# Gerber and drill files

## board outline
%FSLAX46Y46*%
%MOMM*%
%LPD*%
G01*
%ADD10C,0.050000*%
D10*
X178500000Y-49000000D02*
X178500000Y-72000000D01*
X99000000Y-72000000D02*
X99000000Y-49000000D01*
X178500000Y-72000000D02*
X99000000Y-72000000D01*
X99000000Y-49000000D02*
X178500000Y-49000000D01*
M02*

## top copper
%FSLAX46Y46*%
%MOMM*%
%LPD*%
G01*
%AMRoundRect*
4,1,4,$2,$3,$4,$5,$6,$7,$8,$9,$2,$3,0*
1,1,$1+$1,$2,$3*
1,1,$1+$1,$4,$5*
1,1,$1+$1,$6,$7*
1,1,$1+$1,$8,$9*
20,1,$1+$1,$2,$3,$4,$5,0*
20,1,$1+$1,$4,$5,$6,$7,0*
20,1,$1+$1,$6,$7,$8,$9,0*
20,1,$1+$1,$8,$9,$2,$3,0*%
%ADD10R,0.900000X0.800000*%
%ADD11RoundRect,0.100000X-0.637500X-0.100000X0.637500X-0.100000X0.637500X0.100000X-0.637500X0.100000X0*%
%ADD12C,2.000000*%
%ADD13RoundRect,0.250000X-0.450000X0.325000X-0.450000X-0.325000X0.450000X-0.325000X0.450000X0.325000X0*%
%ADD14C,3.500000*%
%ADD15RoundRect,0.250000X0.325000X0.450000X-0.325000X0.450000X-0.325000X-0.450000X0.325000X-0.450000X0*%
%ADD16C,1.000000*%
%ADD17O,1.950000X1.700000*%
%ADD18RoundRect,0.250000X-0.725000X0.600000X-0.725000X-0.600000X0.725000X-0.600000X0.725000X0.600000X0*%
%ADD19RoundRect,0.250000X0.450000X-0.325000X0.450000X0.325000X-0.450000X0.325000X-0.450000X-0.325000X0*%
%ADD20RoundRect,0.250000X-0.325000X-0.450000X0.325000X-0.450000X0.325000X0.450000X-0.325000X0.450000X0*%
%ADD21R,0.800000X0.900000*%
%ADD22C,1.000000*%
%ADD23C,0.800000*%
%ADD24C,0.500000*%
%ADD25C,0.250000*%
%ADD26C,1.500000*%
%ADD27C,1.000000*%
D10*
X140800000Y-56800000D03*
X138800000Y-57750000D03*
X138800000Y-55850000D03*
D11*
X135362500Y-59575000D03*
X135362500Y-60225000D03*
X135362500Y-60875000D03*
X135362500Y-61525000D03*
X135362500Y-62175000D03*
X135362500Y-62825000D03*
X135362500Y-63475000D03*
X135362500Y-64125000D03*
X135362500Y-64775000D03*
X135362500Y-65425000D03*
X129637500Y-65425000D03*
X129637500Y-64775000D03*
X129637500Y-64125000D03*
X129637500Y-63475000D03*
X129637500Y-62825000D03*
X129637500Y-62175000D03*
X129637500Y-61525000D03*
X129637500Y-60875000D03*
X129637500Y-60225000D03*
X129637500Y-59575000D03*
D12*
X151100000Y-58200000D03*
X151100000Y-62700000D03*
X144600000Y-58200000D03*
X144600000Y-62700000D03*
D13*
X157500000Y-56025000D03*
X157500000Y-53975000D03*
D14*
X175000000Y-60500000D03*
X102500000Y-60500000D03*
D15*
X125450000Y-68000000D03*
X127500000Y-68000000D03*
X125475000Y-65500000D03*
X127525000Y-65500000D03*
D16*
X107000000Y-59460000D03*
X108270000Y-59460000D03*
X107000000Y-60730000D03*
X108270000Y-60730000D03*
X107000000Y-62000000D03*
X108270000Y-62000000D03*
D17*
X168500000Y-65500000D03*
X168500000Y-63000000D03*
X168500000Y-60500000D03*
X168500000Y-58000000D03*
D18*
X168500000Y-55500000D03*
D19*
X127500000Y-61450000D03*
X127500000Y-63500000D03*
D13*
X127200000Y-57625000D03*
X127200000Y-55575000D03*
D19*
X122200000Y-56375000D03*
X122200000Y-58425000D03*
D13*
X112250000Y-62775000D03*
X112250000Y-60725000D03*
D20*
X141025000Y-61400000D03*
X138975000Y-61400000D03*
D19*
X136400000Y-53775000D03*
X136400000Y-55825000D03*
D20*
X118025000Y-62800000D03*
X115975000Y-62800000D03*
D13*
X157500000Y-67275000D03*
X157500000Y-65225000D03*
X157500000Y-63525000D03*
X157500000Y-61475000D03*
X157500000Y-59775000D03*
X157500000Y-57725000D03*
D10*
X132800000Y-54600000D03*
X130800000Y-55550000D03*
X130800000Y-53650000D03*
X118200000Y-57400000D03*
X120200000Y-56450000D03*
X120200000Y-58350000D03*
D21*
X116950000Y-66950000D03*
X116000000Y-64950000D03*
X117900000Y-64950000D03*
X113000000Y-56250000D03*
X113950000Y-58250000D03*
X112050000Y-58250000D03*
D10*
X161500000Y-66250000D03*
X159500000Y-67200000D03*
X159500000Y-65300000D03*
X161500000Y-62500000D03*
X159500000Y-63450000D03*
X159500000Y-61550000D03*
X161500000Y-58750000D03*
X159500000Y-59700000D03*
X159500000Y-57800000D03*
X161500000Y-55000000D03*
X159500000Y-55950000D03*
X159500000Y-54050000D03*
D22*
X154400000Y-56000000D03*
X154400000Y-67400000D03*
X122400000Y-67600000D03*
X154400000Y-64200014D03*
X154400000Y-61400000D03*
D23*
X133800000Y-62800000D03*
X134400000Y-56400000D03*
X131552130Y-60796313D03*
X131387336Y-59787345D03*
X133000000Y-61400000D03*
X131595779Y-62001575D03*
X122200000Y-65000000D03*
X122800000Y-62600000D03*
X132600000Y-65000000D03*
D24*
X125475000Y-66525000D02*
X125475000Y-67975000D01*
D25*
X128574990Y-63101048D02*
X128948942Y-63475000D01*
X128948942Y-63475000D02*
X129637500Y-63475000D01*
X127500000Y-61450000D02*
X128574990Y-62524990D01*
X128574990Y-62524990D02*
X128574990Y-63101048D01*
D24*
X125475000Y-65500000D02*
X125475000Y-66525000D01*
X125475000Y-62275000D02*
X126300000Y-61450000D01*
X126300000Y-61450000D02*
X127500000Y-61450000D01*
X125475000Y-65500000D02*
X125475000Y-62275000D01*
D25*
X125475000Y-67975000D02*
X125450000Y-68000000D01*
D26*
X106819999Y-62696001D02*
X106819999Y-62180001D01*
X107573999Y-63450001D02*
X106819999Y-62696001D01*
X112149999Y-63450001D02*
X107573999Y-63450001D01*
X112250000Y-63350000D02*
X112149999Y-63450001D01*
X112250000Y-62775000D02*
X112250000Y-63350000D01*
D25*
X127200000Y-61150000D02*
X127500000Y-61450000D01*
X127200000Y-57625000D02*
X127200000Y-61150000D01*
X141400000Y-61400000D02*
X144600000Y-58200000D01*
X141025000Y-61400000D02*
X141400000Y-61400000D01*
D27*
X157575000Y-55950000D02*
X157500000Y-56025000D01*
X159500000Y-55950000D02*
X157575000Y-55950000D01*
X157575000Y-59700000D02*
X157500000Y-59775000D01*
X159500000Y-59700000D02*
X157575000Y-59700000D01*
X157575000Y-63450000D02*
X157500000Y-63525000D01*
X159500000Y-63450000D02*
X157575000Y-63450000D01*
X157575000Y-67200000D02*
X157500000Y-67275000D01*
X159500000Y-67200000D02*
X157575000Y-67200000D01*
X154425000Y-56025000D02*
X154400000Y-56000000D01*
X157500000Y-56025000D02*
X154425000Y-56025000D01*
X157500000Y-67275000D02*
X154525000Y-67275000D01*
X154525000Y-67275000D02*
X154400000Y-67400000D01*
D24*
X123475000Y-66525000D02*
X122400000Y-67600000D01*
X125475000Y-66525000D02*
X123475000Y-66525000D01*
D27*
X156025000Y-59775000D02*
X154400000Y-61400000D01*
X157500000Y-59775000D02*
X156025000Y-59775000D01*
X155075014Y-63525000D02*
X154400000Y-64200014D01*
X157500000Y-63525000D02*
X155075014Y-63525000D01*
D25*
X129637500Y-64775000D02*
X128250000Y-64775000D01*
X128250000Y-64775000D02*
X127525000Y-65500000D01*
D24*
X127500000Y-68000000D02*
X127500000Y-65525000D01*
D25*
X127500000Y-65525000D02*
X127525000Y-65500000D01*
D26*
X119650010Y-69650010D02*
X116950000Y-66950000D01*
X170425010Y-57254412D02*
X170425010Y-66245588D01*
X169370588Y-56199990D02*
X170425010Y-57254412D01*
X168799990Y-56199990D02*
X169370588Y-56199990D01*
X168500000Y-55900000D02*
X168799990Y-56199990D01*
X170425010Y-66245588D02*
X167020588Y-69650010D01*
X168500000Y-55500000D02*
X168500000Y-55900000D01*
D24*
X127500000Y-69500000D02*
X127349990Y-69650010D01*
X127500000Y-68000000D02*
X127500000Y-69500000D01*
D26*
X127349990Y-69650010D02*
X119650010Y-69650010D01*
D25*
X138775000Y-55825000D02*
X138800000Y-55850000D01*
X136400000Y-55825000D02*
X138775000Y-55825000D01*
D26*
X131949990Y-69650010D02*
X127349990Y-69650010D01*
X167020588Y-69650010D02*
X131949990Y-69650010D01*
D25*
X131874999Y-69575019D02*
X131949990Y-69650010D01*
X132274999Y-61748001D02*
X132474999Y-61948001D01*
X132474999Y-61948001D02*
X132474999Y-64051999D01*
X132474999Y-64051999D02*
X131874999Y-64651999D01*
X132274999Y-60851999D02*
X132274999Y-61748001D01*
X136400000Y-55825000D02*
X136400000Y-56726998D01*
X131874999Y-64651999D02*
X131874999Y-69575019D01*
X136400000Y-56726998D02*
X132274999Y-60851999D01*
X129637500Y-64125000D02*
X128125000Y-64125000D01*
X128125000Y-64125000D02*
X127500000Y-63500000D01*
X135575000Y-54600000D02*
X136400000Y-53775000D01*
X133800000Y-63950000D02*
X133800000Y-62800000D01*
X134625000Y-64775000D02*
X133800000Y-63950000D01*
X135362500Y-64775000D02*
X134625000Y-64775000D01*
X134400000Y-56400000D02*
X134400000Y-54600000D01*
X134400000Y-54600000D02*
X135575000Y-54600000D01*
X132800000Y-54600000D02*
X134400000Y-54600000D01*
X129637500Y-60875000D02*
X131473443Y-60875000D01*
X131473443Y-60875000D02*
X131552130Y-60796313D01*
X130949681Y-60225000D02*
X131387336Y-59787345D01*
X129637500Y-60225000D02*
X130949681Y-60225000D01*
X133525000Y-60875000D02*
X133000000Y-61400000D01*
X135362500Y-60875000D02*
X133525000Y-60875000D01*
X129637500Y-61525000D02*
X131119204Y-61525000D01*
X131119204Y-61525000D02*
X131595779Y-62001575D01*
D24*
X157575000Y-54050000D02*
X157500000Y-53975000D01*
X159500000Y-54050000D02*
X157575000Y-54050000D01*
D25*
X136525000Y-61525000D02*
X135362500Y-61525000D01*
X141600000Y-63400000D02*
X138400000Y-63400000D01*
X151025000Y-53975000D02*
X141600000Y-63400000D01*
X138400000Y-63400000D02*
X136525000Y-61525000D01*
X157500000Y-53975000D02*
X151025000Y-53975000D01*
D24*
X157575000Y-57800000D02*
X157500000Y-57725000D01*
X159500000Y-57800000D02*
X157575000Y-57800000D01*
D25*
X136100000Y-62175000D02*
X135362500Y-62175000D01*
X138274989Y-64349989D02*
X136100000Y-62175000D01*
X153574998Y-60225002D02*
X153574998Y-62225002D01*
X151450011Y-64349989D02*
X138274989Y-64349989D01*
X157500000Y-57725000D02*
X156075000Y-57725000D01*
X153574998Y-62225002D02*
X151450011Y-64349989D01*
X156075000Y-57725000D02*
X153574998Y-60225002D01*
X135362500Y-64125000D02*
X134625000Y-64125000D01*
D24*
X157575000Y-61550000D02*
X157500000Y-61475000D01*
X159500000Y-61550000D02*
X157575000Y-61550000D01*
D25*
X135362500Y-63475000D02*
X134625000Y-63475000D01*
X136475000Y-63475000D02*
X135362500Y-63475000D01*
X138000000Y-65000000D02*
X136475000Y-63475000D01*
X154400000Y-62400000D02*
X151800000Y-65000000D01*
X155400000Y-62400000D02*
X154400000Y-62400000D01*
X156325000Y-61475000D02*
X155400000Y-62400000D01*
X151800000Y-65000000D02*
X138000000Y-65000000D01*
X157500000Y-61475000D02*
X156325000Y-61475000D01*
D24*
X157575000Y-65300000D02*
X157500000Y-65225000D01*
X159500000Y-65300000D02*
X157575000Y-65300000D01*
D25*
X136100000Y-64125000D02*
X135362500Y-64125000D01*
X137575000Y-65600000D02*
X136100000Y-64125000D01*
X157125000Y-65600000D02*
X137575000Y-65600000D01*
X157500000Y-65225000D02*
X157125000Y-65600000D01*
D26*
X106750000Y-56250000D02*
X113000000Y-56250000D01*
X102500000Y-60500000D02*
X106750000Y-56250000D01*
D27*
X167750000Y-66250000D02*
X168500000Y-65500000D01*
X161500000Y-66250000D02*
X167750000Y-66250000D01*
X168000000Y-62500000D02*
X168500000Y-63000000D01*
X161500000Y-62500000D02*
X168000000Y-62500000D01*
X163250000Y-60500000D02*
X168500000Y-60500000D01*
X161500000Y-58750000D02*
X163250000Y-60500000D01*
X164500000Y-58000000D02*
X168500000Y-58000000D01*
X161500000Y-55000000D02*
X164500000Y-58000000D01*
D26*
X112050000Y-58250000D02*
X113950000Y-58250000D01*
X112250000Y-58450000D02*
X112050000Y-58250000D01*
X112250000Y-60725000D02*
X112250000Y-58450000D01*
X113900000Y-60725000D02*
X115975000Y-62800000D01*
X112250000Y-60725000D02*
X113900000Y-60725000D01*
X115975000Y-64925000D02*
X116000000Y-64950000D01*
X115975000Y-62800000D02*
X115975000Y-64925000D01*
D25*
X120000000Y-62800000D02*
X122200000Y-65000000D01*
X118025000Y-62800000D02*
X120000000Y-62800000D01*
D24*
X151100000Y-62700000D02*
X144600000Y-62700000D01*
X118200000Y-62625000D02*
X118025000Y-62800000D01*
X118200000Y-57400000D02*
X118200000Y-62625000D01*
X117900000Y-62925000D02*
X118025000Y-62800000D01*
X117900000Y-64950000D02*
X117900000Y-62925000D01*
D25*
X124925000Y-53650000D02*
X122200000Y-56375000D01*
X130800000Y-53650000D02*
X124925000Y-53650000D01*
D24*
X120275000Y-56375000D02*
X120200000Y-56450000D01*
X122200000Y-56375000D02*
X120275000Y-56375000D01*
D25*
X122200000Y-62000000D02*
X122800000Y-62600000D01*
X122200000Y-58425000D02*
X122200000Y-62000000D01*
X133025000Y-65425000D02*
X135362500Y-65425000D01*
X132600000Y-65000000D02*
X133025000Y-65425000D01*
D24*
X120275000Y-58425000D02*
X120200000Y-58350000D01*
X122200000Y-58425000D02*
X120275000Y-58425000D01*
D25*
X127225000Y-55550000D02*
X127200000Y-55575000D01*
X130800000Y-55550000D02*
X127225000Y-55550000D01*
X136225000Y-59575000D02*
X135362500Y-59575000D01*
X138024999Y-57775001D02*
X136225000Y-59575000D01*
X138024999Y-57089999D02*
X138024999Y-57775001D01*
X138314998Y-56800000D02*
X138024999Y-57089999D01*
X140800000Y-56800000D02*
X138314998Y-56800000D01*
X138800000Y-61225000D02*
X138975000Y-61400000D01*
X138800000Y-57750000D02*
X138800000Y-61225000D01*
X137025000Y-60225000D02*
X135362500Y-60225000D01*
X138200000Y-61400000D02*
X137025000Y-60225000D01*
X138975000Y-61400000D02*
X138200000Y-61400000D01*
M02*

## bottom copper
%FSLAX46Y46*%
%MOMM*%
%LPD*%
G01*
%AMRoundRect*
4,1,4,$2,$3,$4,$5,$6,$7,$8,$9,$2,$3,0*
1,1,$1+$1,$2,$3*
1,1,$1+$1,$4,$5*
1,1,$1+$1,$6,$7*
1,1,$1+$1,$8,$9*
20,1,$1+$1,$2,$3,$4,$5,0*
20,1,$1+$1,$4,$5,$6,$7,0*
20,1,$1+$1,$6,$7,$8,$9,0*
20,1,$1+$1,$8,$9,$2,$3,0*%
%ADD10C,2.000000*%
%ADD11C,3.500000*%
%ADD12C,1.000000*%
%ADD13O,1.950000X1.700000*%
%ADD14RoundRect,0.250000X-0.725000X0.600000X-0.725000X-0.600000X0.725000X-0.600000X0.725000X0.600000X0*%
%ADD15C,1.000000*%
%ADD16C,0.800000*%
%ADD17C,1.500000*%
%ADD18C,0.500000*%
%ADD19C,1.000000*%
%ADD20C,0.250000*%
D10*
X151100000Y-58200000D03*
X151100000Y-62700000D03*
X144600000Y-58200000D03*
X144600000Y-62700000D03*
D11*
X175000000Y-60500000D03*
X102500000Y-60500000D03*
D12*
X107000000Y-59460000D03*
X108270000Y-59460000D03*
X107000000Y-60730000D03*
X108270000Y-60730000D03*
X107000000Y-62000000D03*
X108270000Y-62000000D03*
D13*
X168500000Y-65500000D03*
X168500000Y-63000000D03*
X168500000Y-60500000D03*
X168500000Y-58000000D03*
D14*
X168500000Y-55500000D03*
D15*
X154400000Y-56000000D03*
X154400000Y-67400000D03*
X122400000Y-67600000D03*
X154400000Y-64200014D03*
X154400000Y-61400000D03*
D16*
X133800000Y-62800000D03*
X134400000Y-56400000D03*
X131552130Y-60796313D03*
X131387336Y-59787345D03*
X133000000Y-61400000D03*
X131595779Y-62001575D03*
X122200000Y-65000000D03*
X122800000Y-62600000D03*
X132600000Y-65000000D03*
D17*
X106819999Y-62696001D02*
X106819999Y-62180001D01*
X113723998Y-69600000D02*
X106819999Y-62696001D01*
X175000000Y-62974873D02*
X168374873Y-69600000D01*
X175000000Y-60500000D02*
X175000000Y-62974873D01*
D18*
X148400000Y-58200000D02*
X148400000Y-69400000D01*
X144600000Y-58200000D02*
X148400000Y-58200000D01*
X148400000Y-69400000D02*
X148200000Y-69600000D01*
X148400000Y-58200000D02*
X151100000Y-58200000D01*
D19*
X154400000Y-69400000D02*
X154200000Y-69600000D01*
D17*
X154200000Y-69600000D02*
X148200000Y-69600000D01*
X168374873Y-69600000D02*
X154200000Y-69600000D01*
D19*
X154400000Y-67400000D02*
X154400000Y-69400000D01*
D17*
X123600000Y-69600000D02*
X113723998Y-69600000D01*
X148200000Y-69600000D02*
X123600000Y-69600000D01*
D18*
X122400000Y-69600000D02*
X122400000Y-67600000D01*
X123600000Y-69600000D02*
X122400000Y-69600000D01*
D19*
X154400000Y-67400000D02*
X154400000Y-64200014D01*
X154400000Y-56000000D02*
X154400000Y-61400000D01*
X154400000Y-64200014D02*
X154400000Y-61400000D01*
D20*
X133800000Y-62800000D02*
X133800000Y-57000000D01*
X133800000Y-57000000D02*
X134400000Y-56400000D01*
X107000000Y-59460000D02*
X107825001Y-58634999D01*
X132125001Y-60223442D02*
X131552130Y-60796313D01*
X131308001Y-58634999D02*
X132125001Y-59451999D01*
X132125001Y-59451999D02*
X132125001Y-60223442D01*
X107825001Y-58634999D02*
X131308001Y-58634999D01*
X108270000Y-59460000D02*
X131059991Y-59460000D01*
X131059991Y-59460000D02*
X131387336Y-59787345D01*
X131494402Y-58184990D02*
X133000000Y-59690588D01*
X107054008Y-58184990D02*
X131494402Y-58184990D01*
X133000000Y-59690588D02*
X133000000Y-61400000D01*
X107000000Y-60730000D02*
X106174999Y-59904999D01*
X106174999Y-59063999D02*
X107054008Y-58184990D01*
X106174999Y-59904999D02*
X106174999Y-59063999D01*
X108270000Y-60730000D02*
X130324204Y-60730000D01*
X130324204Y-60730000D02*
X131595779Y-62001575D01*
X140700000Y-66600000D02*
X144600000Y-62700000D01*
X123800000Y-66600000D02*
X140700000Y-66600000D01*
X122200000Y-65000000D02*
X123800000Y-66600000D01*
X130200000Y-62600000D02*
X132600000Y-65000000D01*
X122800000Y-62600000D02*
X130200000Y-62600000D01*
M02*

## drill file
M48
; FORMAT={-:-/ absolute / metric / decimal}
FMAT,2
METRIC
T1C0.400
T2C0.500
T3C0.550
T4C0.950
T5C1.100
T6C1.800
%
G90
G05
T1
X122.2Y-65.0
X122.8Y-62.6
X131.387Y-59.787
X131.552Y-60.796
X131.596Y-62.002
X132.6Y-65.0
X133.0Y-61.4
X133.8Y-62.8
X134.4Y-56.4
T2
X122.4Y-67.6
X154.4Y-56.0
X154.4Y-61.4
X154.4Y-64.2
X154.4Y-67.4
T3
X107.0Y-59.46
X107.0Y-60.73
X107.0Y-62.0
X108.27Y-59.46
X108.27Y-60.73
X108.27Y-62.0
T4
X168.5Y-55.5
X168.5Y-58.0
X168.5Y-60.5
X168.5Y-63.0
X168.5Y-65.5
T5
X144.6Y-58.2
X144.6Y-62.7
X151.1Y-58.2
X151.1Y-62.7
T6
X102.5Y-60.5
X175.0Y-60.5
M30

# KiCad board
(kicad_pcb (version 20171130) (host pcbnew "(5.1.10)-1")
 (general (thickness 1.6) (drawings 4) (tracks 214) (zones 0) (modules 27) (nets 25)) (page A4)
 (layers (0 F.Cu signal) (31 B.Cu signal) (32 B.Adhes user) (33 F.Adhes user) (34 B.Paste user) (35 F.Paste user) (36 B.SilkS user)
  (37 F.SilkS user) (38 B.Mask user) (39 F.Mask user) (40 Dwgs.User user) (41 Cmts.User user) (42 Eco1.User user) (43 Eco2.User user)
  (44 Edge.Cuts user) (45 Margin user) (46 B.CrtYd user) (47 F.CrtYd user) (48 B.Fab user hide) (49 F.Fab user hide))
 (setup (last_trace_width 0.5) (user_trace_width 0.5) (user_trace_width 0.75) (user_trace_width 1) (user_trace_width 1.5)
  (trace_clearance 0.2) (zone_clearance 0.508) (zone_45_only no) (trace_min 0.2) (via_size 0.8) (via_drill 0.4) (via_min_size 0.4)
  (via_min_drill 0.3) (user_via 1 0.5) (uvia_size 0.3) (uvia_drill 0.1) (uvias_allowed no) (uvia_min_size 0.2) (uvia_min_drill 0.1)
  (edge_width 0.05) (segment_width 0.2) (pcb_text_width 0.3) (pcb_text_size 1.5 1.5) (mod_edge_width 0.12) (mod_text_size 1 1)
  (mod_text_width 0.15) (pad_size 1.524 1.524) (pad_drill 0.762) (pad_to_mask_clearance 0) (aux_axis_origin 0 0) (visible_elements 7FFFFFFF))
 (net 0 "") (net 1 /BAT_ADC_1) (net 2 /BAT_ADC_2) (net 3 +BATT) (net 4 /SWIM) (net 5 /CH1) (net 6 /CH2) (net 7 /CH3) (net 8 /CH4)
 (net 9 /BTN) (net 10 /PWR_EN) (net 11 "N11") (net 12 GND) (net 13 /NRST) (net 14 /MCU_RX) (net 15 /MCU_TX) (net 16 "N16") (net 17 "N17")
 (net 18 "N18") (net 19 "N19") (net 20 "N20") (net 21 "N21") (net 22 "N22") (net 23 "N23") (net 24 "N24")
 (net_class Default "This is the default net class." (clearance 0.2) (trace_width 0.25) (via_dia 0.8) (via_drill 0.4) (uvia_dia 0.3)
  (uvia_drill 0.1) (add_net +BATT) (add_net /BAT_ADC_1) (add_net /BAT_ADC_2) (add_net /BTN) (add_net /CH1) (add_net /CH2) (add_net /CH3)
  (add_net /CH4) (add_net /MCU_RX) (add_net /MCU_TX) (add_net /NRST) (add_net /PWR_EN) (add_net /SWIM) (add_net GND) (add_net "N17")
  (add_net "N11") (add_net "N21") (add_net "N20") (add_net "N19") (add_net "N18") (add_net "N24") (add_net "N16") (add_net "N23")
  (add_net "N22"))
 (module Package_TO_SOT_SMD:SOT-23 (layer F.Cu) (at 139.8 56.8)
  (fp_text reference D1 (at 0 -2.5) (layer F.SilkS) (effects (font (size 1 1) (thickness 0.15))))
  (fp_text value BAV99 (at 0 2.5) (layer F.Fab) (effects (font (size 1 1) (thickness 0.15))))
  (pad 3 smd rect (at 1 0) (size 0.9 0.8) (layers F.Cu F.Paste F.Mask) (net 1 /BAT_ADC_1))
  (pad 2 smd rect (at -1 0.95) (size 0.9 0.8) (layers F.Cu F.Paste F.Mask) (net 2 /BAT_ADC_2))
  (pad 1 smd rect (at -1 -0.95) (size 0.9 0.8) (layers F.Cu F.Paste F.Mask) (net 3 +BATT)))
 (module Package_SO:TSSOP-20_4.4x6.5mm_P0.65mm (layer F.Cu) (at 132.5 62.5)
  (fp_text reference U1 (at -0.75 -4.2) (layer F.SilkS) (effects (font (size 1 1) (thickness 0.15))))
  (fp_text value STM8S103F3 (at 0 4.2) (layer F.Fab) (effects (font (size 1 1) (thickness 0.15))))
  (pad 20 smd roundrect (at 2.8625 -2.925) (size 1.475 0.4) (layers F.Cu F.Paste F.Mask) (roundrect_rratio 0.25) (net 1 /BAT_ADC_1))
  (pad 19 smd roundrect (at 2.8625 -2.275) (size 1.475 0.4) (layers F.Cu F.Paste F.Mask) (roundrect_rratio 0.25) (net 2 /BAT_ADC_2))
  (pad 18 smd roundrect (at 2.8625 -1.625) (size 1.475 0.4) (layers F.Cu F.Paste F.Mask) (roundrect_rratio 0.25) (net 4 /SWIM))
  (pad 17 smd roundrect (at 2.8625 -0.975) (size 1.475 0.4) (layers F.Cu F.Paste F.Mask) (roundrect_rratio 0.25) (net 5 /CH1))
  (pad 16 smd roundrect (at 2.8625 -0.325) (size 1.475 0.4) (layers F.Cu F.Paste F.Mask) (roundrect_rratio 0.25) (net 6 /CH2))
  (pad 15 smd roundrect (at 2.8625 0.325) (size 1.475 0.4) (layers F.Cu F.Paste F.Mask) (roundrect_rratio 0.25))
  (pad 14 smd roundrect (at 2.8625 0.975) (size 1.475 0.4) (layers F.Cu F.Paste F.Mask) (roundrect_rratio 0.25) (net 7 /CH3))
  (pad 13 smd roundrect (at 2.8625 1.625) (size 1.475 0.4) (layers F.Cu F.Paste F.Mask) (roundrect_rratio 0.25) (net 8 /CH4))
  (pad 12 smd roundrect (at 2.8625 2.275) (size 1.475 0.4) (layers F.Cu F.Paste F.Mask) (roundrect_rratio 0.25) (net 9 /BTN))
  (pad 11 smd roundrect (at 2.8625 2.925) (size 1.475 0.4) (layers F.Cu F.Paste F.Mask) (roundrect_rratio 0.25) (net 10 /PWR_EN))
  (pad 10 smd roundrect (at -2.8625 2.925) (size 1.475 0.4) (layers F.Cu F.Paste F.Mask) (roundrect_rratio 0.25))
  (pad 9 smd roundrect (at -2.8625 2.275) (size 1.475 0.4) (layers F.Cu F.Paste F.Mask) (roundrect_rratio 0.25) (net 3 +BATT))
  (pad 8 smd roundrect (at -2.8625 1.625) (size 1.475 0.4) (layers F.Cu F.Paste F.Mask) (roundrect_rratio 0.25) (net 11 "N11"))
  (pad 7 smd roundrect (at -2.8625 0.975) (size 1.475 0.4) (layers F.Cu F.Paste F.Mask) (roundrect_rratio 0.25) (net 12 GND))
  (pad 6 smd roundrect (at -2.8625 0.325) (size 1.475 0.4) (layers F.Cu F.Paste F.Mask) (roundrect_rratio 0.25))
  (pad 5 smd roundrect (at -2.8625 -0.325) (size 1.475 0.4) (layers F.Cu F.Paste F.Mask) (roundrect_rratio 0.25))
  (pad 4 smd roundrect (at -2.8625 -0.975) (size 1.475 0.4) (layers F.Cu F.Paste F.Mask) (roundrect_rratio 0.25) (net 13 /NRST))
  (pad 3 smd roundrect (at -2.8625 -1.625) (size 1.475 0.4) (layers F.Cu F.Paste F.Mask) (roundrect_rratio 0.25) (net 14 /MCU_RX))
  (pad 2 smd roundrect (at -2.8625 -2.275) (size 1.475 0.4) (layers F.Cu F.Paste F.Mask) (roundrect_rratio 0.25) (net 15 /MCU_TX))
  (pad 1 smd roundrect (at -2.8625 -2.925) (size 1.475 0.4) (layers F.Cu F.Paste F.Mask) (roundrect_rratio 0.25)))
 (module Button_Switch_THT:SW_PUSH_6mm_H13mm (layer F.Cu) (at 144.6 58.2)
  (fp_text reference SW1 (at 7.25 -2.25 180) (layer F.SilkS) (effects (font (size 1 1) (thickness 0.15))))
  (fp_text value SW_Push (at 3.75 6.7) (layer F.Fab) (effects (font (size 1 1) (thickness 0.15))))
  (pad 1 thru_hole circle (at 6.5 0 90) (size 2 2) (drill 1.1) (layers *.Cu *.Mask) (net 12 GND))
  (pad 2 thru_hole circle (at 6.5 4.5 90) (size 2 2) (drill 1.1) (layers *.Cu *.Mask) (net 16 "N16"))
  (pad 1 thru_hole circle (at 0 0 90) (size 2 2) (drill 1.1) (layers *.Cu *.Mask) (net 12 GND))
  (pad 2 thru_hole circle (at 0 4.5 90) (size 2 2) (drill 1.1) (layers *.Cu *.Mask) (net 16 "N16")))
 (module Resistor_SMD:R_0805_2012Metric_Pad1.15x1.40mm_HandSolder (layer F.Cu) (at 157.5 55 270)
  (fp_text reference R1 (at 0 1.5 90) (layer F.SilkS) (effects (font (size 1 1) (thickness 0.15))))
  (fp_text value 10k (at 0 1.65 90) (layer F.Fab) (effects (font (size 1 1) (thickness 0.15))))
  (pad 2 smd roundrect (at 1.025 0 270) (size 1.15 1.4) (layers F.Cu F.Paste F.Mask) (roundrect_rratio 0.217391) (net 12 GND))
  (pad 1 smd roundrect (at -1.025 0 270) (size 1.15 1.4) (layers F.Cu F.Paste F.Mask) (roundrect_rratio 0.217391) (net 5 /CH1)))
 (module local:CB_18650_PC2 (layer B.Cu) (at 100 71)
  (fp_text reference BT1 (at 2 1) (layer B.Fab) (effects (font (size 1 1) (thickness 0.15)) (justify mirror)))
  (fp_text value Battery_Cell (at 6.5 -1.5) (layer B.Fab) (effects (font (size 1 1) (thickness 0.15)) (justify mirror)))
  (pad 2 thru_hole circle (at 75 -10.5) (size 3.5 3.5) (drill 1.8) (layers *.Cu *.Mask) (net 12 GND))
  (pad 1 thru_hole circle (at 2.5 -10.5) (size 3.5 3.5) (drill 1.8) (layers *.Cu *.Mask) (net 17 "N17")))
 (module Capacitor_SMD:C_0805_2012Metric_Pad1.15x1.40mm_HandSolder (layer F.Cu) (at 126.475 68 180)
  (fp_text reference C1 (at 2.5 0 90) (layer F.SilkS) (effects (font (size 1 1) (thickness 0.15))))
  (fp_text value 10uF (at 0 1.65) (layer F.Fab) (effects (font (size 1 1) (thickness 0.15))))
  (pad 2 smd roundrect (at 1.025 0 180) (size 1.15 1.4) (layers F.Cu F.Paste F.Mask) (roundrect_rratio 0.217391) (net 12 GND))
  (pad 1 smd roundrect (at -1.025 0 180) (size 1.15 1.4) (layers F.Cu F.Paste F.Mask) (roundrect_rratio 0.217391) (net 3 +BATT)))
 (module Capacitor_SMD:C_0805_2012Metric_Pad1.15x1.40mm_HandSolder (layer F.Cu) (at 126.5 65.5 180)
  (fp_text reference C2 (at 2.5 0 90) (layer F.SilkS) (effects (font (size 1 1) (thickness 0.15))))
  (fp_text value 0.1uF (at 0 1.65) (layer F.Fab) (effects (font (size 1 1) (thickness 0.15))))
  (pad 2 smd roundrect (at 1.025 0 180) (size 1.15 1.4) (layers F.Cu F.Paste F.Mask) (roundrect_rratio 0.217391) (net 12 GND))
  (pad 1 smd roundrect (at -1.025 0 180) (size 1.15 1.4) (layers F.Cu F.Paste F.Mask) (roundrect_rratio 0.217391) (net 3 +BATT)))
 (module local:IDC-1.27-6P (layer F.Cu) (at 107 62 90)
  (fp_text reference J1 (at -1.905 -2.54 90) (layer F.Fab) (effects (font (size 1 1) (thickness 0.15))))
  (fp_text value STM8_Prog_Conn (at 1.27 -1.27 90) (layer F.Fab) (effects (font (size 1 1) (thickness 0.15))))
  (pad 6 thru_hole circle (at 2.54 0 90) (size 1 1) (drill 0.55) (layers *.Cu *.Mask) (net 14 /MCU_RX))
  (pad 5 thru_hole circle (at 2.54 1.27 90) (size 1 1) (drill 0.55) (layers *.Cu *.Mask) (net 15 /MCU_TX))
  (pad 4 thru_hole circle (at 1.27 0 90) (size 1 1) (drill 0.55) (layers *.Cu *.Mask) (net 4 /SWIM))
  (pad 3 thru_hole circle (at 1.27 1.27 90) (size 1 1) (drill 0.55) (layers *.Cu *.Mask) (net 13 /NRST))
  (pad 2 thru_hole circle (at 0 0 90) (size 1 1) (drill 0.55) (layers *.Cu *.Mask) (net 12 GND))
  (pad 1 thru_hole circle (at 0 1.27 90) (size 1 1) (drill 0.55) (layers *.Cu *.Mask)))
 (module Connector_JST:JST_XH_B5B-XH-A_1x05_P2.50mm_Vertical (layer F.Cu) (at 168.5 55.5 270)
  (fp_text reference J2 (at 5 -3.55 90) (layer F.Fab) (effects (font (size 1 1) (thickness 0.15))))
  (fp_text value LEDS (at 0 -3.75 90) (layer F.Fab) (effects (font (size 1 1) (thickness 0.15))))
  (pad 5 thru_hole oval (at 10 0 270) (size 1.7 1.95) (drill 0.95) (layers *.Cu *.Mask) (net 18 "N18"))
  (pad 4 thru_hole oval (at 7.5 0 270) (size 1.7 1.95) (drill 0.95) (layers *.Cu *.Mask) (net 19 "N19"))
  (pad 3 thru_hole oval (at 5 0 270) (size 1.7 1.95) (drill 0.95) (layers *.Cu *.Mask) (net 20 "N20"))
  (pad 2 thru_hole oval (at 2.5 0 270) (size 1.7 1.95) (drill 0.95) (layers *.Cu *.Mask) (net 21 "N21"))
  (pad 1 thru_hole roundrect (at 0 0 270) (size 1.7 1.95) (drill 0.95) (layers *.Cu *.Mask) (roundrect_rratio 0.147059) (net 3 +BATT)))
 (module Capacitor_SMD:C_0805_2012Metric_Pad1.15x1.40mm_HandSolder (layer F.Cu) (at 127.5 62.475 90)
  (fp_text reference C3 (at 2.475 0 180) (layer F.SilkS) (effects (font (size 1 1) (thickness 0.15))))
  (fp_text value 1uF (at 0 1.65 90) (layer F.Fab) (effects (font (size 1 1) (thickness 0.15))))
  (pad 2 smd roundrect (at 1.025 0 90) (size 1.15 1.4) (layers F.Cu F.Paste F.Mask) (roundrect_rratio 0.217391) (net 12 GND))
  (pad 1 smd roundrect (at -1.025 0 90) (size 1.15 1.4) (layers F.Cu F.Paste F.Mask) (roundrect_rratio 0.217391) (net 11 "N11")))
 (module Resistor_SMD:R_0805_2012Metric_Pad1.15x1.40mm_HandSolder (layer F.Cu) (at 127.2 56.6 270)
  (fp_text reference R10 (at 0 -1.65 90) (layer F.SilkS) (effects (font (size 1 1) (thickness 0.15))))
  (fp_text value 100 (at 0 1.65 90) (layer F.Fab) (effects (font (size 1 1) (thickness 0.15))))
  (pad 2 smd roundrect (at 1.025 0 270) (size 1.15 1.4) (layers F.Cu F.Paste F.Mask) (roundrect_rratio 0.217391) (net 12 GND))
  (pad 1 smd roundrect (at -1.025 0 270) (size 1.15 1.4) (layers F.Cu F.Paste F.Mask) (roundrect_rratio 0.217391) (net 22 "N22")))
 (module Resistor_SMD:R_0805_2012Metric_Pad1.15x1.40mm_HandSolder (layer F.Cu) (at 122.2 57.4 90)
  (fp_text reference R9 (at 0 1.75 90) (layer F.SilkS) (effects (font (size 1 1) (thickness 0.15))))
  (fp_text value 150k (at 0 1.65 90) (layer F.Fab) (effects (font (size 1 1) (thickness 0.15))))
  (pad 2 smd roundrect (at 1.025 0 90) (size 1.15 1.4) (layers F.Cu F.Paste F.Mask) (roundrect_rratio 0.217391) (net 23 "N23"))
  (pad 1 smd roundrect (at -1.025 0 90) (size 1.15 1.4) (layers F.Cu F.Paste F.Mask) (roundrect_rratio 0.217391) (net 10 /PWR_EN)))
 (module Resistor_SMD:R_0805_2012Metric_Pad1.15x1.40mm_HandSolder (layer F.Cu) (at 112.25 61.75 270)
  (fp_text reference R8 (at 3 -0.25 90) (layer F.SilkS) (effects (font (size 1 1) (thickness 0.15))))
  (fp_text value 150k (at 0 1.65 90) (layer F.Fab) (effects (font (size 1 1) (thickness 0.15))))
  (pad 2 smd roundrect (at 1.025 0 270) (size 1.15 1.4) (layers F.Cu F.Paste F.Mask) (roundrect_rratio 0.217391) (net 12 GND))
  (pad 1 smd roundrect (at -1.025 0 270) (size 1.15 1.4) (layers F.Cu F.Paste F.Mask) (roundrect_rratio 0.217391) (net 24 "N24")))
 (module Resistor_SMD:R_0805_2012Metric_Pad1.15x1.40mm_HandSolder (layer F.Cu) (at 140 61.4)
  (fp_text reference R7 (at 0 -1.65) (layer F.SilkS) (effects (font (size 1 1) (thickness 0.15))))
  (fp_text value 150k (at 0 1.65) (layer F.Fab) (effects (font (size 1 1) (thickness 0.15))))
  (pad 2 smd roundrect (at 1.025 0) (size 1.15 1.4) (layers F.Cu F.Paste F.Mask) (roundrect_rratio 0.217391) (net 12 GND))
  (pad 1 smd roundrect (at -1.025 0) (size 1.15 1.4) (layers F.Cu F.Paste F.Mask) (roundrect_rratio 0.217391) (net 2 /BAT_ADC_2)))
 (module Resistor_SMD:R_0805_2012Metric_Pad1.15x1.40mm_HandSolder (layer F.Cu) (at 136.4 54.8 90)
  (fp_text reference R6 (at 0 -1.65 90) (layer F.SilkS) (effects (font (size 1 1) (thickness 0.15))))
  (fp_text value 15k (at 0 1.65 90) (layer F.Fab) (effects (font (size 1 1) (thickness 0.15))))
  (pad 2 smd roundrect (at 1.025 0 90) (size 1.15 1.4) (layers F.Cu F.Paste F.Mask) (roundrect_rratio 0.217391) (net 9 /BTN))
  (pad 1 smd roundrect (at -1.025 0 90) (size 1.15 1.4) (layers F.Cu F.Paste F.Mask) (roundrect_rratio 0.217391) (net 3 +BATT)))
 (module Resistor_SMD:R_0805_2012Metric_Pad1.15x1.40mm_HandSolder (layer F.Cu) (at 117 62.8)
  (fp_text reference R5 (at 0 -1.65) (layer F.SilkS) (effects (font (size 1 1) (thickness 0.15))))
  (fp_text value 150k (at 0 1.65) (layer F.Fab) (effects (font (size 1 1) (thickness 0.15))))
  (pad 2 smd roundrect (at 1.025 0) (size 1.15 1.4) (layers F.Cu F.Paste F.Mask) (roundrect_rratio 0.217391) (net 16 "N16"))
  (pad 1 smd roundrect (at -1.025 0) (size 1.15 1.4) (layers F.Cu F.Paste F.Mask) (roundrect_rratio 0.217391) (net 24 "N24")))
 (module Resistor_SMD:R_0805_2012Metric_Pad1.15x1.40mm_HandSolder (layer F.Cu) (at 157.5 66.25 270)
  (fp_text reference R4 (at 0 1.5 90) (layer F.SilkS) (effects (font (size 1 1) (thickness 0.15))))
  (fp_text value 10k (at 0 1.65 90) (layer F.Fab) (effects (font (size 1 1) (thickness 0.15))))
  (pad 2 smd roundrect (at 1.025 0 270) (size 1.15 1.4) (layers F.Cu F.Paste F.Mask) (roundrect_rratio 0.217391) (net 12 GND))
  (pad 1 smd roundrect (at -1.025 0 270) (size 1.15 1.4) (layers F.Cu F.Paste F.Mask) (roundrect_rratio 0.217391) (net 8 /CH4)))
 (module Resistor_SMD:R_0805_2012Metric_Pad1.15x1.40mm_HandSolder (layer F.Cu) (at 157.5 62.5 270)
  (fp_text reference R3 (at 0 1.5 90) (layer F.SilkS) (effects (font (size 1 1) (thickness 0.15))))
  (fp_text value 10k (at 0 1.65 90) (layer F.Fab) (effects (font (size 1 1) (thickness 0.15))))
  (pad 2 smd roundrect (at 1.025 0 270) (size 1.15 1.4) (layers F.Cu F.Paste F.Mask) (roundrect_rratio 0.217391) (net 12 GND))
  (pad 1 smd roundrect (at -1.025 0 270) (size 1.15 1.4) (layers F.Cu F.Paste F.Mask) (roundrect_rratio 0.217391) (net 7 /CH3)))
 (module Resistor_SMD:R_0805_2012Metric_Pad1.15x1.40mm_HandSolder (layer F.Cu) (at 157.5 58.75 270)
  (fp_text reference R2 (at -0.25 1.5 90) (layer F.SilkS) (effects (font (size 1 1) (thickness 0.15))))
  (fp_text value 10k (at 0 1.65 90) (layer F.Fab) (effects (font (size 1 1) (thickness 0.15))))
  (pad 2 smd roundrect (at 1.025 0 270) (size 1.15 1.4) (layers F.Cu F.Paste F.Mask) (roundrect_rratio 0.217391) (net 12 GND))
  (pad 1 smd roundrect (at -1.025 0 270) (size 1.15 1.4) (layers F.Cu F.Paste F.Mask) (roundrect_rratio 0.217391) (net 6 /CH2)))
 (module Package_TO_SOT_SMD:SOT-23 (layer F.Cu) (at 131.8 54.6)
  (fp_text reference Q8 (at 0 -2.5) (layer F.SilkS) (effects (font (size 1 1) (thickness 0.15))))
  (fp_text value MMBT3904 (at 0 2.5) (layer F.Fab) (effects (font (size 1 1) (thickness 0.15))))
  (pad 3 smd rect (at 1 0) (size 0.9 0.8) (layers F.Cu F.Paste F.Mask) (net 9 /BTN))
  (pad 2 smd rect (at -1 0.95) (size 0.9 0.8) (layers F.Cu F.Paste F.Mask) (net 22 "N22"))
  (pad 1 smd rect (at -1 -0.95) (size 0.9 0.8) (layers F.Cu F.Paste F.Mask) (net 23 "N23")))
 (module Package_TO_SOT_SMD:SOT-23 (layer F.Cu) (at 119.2 57.4 180)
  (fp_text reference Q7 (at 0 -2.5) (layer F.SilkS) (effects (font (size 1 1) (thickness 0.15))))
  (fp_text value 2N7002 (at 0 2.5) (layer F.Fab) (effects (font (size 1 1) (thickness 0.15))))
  (pad 3 smd rect (at 1 0 180) (size 0.9 0.8) (layers F.Cu F.Paste F.Mask) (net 16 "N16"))
  (pad 2 smd rect (at -1 0.95 180) (size 0.9 0.8) (layers F.Cu F.Paste F.Mask) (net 23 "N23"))
  (pad 1 smd rect (at -1 -0.95 180) (size 0.9 0.8) (layers F.Cu F.Paste F.Mask) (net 10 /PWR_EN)))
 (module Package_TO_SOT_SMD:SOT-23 (layer F.Cu) (at 116.95 65.95 270)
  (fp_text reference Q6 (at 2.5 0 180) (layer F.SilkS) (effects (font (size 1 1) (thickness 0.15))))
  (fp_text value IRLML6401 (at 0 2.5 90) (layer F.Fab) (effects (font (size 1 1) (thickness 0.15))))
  (pad 3 smd rect (at 1 0 270) (size 0.9 0.8) (layers F.Cu F.Paste F.Mask) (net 3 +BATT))
  (pad 2 smd rect (at -1 0.95 270) (size 0.9 0.8) (layers F.Cu F.Paste F.Mask) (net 24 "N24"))
  (pad 1 smd rect (at -1 -0.95 270) (size 0.9 0.8) (layers F.Cu F.Paste F.Mask) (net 16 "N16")))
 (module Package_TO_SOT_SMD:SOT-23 (layer F.Cu) (at 113 57.25 90)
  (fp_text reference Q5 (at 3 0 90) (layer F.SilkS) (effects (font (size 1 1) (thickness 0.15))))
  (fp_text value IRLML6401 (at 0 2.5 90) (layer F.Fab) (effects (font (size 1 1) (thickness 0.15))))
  (pad 3 smd rect (at 1 0 90) (size 0.9 0.8) (layers F.Cu F.Paste F.Mask) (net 17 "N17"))
  (pad 2 smd rect (at -1 0.95 90) (size 0.9 0.8) (layers F.Cu F.Paste F.Mask) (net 24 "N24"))
  (pad 1 smd rect (at -1 -0.95 90) (size 0.9 0.8) (layers F.Cu F.Paste F.Mask) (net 24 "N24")))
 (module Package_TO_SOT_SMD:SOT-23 (layer F.Cu) (at 160.5 66.25)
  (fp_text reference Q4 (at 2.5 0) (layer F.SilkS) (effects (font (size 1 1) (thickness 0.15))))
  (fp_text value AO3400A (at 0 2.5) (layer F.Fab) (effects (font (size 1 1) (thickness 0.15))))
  (pad 3 smd rect (at 1 0) (size 0.9 0.8) (layers F.Cu F.Paste F.Mask) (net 18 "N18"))
  (pad 2 smd rect (at -1 0.95) (size 0.9 0.8) (layers F.Cu F.Paste F.Mask) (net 12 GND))
  (pad 1 smd rect (at -1 -0.95) (size 0.9 0.8) (layers F.Cu F.Paste F.Mask) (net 8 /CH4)))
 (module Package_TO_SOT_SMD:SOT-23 (layer F.Cu) (at 160.5 62.5)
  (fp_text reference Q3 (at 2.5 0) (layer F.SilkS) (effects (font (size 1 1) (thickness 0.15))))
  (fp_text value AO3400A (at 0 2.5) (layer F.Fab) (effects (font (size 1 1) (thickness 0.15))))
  (pad 3 smd rect (at 1 0) (size 0.9 0.8) (layers F.Cu F.Paste F.Mask) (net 19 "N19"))
  (pad 2 smd rect (at -1 0.95) (size 0.9 0.8) (layers F.Cu F.Paste F.Mask) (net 12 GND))
  (pad 1 smd rect (at -1 -0.95) (size 0.9 0.8) (layers F.Cu F.Paste F.Mask) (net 7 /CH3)))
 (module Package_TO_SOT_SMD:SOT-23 (layer F.Cu) (at 160.5 58.75)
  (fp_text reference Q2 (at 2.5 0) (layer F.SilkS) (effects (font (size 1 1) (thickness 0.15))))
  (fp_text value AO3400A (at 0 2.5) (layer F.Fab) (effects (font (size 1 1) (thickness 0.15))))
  (pad 3 smd rect (at 1 0) (size 0.9 0.8) (layers F.Cu F.Paste F.Mask) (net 20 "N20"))
  (pad 2 smd rect (at -1 0.95) (size 0.9 0.8) (layers F.Cu F.Paste F.Mask) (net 12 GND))
  (pad 1 smd rect (at -1 -0.95) (size 0.9 0.8) (layers F.Cu F.Paste F.Mask) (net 6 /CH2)))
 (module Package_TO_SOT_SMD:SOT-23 (layer F.Cu) (at 160.5 55)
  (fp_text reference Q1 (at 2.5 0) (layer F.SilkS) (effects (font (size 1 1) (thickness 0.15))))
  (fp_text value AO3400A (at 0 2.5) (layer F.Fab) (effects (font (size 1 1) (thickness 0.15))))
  (pad 3 smd rect (at 1 0) (size 0.9 0.8) (layers F.Cu F.Paste F.Mask) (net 21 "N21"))
  (pad 2 smd rect (at -1 0.95) (size 0.9 0.8) (layers F.Cu F.Paste F.Mask) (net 12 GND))
  (pad 1 smd rect (at -1 -0.95) (size 0.9 0.8) (layers F.Cu F.Paste F.Mask) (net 5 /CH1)))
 (gr_line (start 178.5 49) (end 178.5 72) (layer Edge.Cuts) (width 0.05))
 (gr_line (start 99 72) (end 99 49) (layer Edge.Cuts) (width 0.05))
 (gr_line (start 178.5 72) (end 99 72) (layer Edge.Cuts) (width 0.05))
 (gr_line (start 99 49) (end 178.5 49) (layer Edge.Cuts) (width 0.05))
 (segment (start 125.475 66.525) (end 125.475 67.975) (width 0.5) (layer F.Cu) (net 12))
 (segment (start 128.57499 63.101048) (end 128.948942 63.475) (width 0.25) (layer F.Cu) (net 12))
 (segment (start 128.948942 63.475) (end 129.6375 63.475) (width 0.25) (layer F.Cu) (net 12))
 (segment (start 127.5 61.45) (end 128.57499 62.52499) (width 0.25) (layer F.Cu) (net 12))
 (segment (start 128.57499 62.52499) (end 128.57499 63.101048) (width 0.25) (layer F.Cu) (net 12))
 (segment (start 125.475 65.5) (end 125.475 66.525) (width 0.5) (layer F.Cu) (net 12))
 (segment (start 125.475 62.275) (end 126.3 61.45) (width 0.5) (layer F.Cu) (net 12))
 (segment (start 126.3 61.45) (end 127.5 61.45) (width 0.5) (layer F.Cu) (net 12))
 (segment (start 125.475 65.5) (end 125.475 62.275) (width 0.5) (layer F.Cu) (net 12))
 (segment (start 125.475 67.975) (end 125.45 68) (width 0.25) (layer F.Cu) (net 12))
 (segment (start 106.819999 62.696001) (end 106.819999 62.180001) (width 1.5) (layer F.Cu) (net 12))
 (segment (start 107.573999 63.450001) (end 106.819999 62.696001) (width 1.5) (layer F.Cu) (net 12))
 (segment (start 112.149999 63.450001) (end 107.573999 63.450001) (width 1.5) (layer F.Cu) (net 12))
 (segment (start 112.25 63.35) (end 112.149999 63.450001) (width 1.5) (layer F.Cu) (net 12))
 (segment (start 112.25 62.775) (end 112.25 63.35) (width 1.5) (layer F.Cu) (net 12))
 (segment (start 106.819999 62.696001) (end 106.819999 62.180001) (width 1.5) (layer B.Cu) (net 12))
 (segment (start 113.723998 69.6) (end 106.819999 62.696001) (width 1.5) (layer B.Cu) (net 12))
 (segment (start 175 62.974873) (end 168.374873 69.6) (width 1.5) (layer B.Cu) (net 12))
 (segment (start 175 60.5) (end 175 62.974873) (width 1.5) (layer B.Cu) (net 12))
 (segment (start 127.2 61.15) (end 127.5 61.45) (width 0.25) (layer F.Cu) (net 12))
 (segment (start 127.2 57.625) (end 127.2 61.15) (width 0.25) (layer F.Cu) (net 12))
 (segment (start 148.4 58.2) (end 148.4 69.4) (width 0.5) (layer B.Cu) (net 12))
 (segment (start 144.6 58.2) (end 148.4 58.2) (width 0.5) (layer B.Cu) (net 12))
 (segment (start 148.4 69.4) (end 148.2 69.6) (width 0.5) (layer B.Cu) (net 12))
 (segment (start 148.4 58.2) (end 151.1 58.2) (width 0.5) (layer B.Cu) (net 12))
 (segment (start 141.4 61.4) (end 144.6 58.2) (width 0.25) (layer F.Cu) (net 12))
 (segment (start 141.025 61.4) (end 141.4 61.4) (width 0.25) (layer F.Cu) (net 12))
 (segment (start 157.575 55.95) (end 157.5 56.025) (width 1) (layer F.Cu) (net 12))
 (segment (start 159.5 55.95) (end 157.575 55.95) (width 1) (layer F.Cu) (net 12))
 (segment (start 157.575 59.7) (end 157.5 59.775) (width 1) (layer F.Cu) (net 12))
 (segment (start 159.5 59.7) (end 157.575 59.7) (width 1) (layer F.Cu) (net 12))
 (segment (start 157.575 63.45) (end 157.5 63.525) (width 1) (layer F.Cu) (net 12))
 (segment (start 159.5 63.45) (end 157.575 63.45) (width 1) (layer F.Cu) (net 12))
 (segment (start 157.575 67.2) (end 157.5 67.275) (width 1) (layer F.Cu) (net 12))
 (segment (start 159.5 67.2) (end 157.575 67.2) (width 1) (layer F.Cu) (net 12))
 (via (at 154.4 56) (size 1) (drill 0.5) (layers F.Cu B.Cu) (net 12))
 (segment (start 154.425 56.025) (end 154.4 56) (width 1) (layer F.Cu) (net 12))
 (segment (start 157.5 56.025) (end 154.425 56.025) (width 1) (layer F.Cu) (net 12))
 (segment (start 154.4 69.4) (end 154.2 69.6) (width 1) (layer B.Cu) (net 12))
 (segment (start 154.2 69.6) (end 148.2 69.6) (width 1.5) (layer B.Cu) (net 12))
 (segment (start 168.374873 69.6) (end 154.2 69.6) (width 1.5) (layer B.Cu) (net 12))
 (segment (start 157.5 67.275) (end 154.525 67.275) (width 1) (layer F.Cu) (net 12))
 (via (at 154.4 67.4) (size 1) (drill 0.5) (layers F.Cu B.Cu) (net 12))
 (segment (start 154.4 67.4) (end 154.4 69.4) (width 1) (layer B.Cu) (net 12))
 (segment (start 154.525 67.275) (end 154.4 67.4) (width 1) (layer F.Cu) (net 12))
 (segment (start 123.6 69.6) (end 113.723998 69.6) (width 1.5) (layer B.Cu) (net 12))
 (segment (start 148.2 69.6) (end 123.6 69.6) (width 1.5) (layer B.Cu) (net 12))
 (segment (start 123.475 66.525) (end 122.4 67.6) (width 0.5) (layer F.Cu) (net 12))
 (segment (start 125.475 66.525) (end 123.475 66.525) (width 0.5) (layer F.Cu) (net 12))
 (via (at 122.4 67.6) (size 1) (drill 0.5) (layers F.Cu B.Cu) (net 12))
 (segment (start 122.4 69.6) (end 122.4 67.6) (width 0.5) (layer B.Cu) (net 12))
 (segment (start 123.6 69.6) (end 122.4 69.6) (width 0.5) (layer B.Cu) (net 12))
 (via (at 154.4 64.200014) (size 1) (drill 0.5) (layers F.Cu B.Cu) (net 12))
 (segment (start 154.4 67.4) (end 154.4 64.200014) (width 1) (layer B.Cu) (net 12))
 (segment (start 156.025 59.775) (end 154.4 61.4) (width 1) (layer F.Cu) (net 12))
 (segment (start 154.4 56) (end 154.4 61.4) (width 1) (layer B.Cu) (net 12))
 (segment (start 157.5 59.775) (end 156.025 59.775) (width 1) (layer F.Cu) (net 12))
 (segment (start 154.4 64.200014) (end 154.4 61.4) (width 1) (layer B.Cu) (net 12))
 (via (at 154.4 61.4) (size 1) (drill 0.5) (layers F.Cu B.Cu) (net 12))
 (segment (start 155.075014 63.525) (end 154.4 64.200014) (width 1) (layer F.Cu) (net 12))
 (segment (start 157.5 63.525) (end 155.075014 63.525) (width 1) (layer F.Cu) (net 12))
 (segment (start 129.6375 64.775) (end 128.25 64.775) (width 0.25) (layer F.Cu) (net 3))
 (segment (start 128.25 64.775) (end 127.525 65.5) (width 0.25) (layer F.Cu) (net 3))
 (segment (start 127.5 68) (end 127.5 65.525) (width 0.5) (layer F.Cu) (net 3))
 (segment (start 127.5 65.525) (end 127.525 65.5) (width 0.25) (layer F.Cu) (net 3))
 (segment (start 119.65001 69.65001) (end 116.95 66.95) (width 1.5) (layer F.Cu) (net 3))
 (segment (start 170.42501 57.254412) (end 170.42501 66.245588) (width 1.5) (layer F.Cu) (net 3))
 (segment (start 169.370588 56.19999) (end 170.42501 57.254412) (width 1.5) (layer F.Cu) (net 3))
 (segment (start 168.79999 56.19999) (end 169.370588 56.19999) (width 1.5) (layer F.Cu) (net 3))
 (segment (start 168.5 55.9) (end 168.79999 56.19999) (width 1.5) (layer F.Cu) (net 3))
 (segment (start 170.42501 66.245588) (end 167.020588 69.65001) (width 1.5) (layer F.Cu) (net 3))
 (segment (start 168.5 55.5) (end 168.5 55.9) (width 1.5) (layer F.Cu) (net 3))
 (segment (start 127.5 69.5) (end 127.34999 69.65001) (width 0.5) (layer F.Cu) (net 3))
 (segment (start 127.5 68) (end 127.5 69.5) (width 0.5) (layer F.Cu) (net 3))
 (segment (start 127.34999 69.65001) (end 119.65001 69.65001) (width 1.5) (layer F.Cu) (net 3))
 (segment (start 138.775 55.825) (end 138.8 55.85) (width 0.25) (layer F.Cu) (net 3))
 (segment (start 136.4 55.825) (end 138.775 55.825) (width 0.25) (layer F.Cu) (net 3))
 (segment (start 131.94999 69.65001) (end 127.34999 69.65001) (width 1.5) (layer F.Cu) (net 3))
 (segment (start 167.020588 69.65001) (end 131.94999 69.65001) (width 1.5) (layer F.Cu) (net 3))
 (segment (start 131.874999 69.575019) (end 131.94999 69.65001) (width 0.25) (layer F.Cu) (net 3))
 (segment (start 132.274999 61.748001) (end 132.474999 61.948001) (width 0.25) (layer F.Cu) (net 3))
 (segment (start 132.474999 61.948001) (end 132.474999 64.051999) (width 0.25) (layer F.Cu) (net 3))
 (segment (start 132.474999 64.051999) (end 131.874999 64.651999) (width 0.25) (layer F.Cu) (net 3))
 (segment (start 132.274999 60.851999) (end 132.274999 61.748001) (width 0.25) (layer F.Cu) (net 3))
 (segment (start 136.4 55.825) (end 136.4 56.726998) (width 0.25) (layer F.Cu) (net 3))
 (segment (start 131.874999 64.651999) (end 131.874999 69.575019) (width 0.25) (layer F.Cu) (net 3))
 (segment (start 136.4 56.726998) (end 132.274999 60.851999) (width 0.25) (layer F.Cu) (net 3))
 (segment (start 129.6375 64.125) (end 128.125 64.125) (width 0.25) (layer F.Cu) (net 11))
 (segment (start 128.125 64.125) (end 127.5 63.5) (width 0.25) (layer F.Cu) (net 11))
 (segment (start 135.575 54.6) (end 136.4 53.775) (width 0.25) (layer F.Cu) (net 9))
 (via (at 133.8 62.8) (size 0.8) (drill 0.4) (layers F.Cu B.Cu) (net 9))
 (segment (start 133.8 63.95) (end 133.8 62.8) (width 0.25) (layer F.Cu) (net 9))
 (segment (start 134.625 64.775) (end 133.8 63.95) (width 0.25) (layer F.Cu) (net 9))
 (segment (start 135.3625 64.775) (end 134.625 64.775) (width 0.25) (layer F.Cu) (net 9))
 (segment (start 133.8 62.8) (end 133.8 57) (width 0.25) (layer B.Cu) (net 9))
 (via (at 134.4 56.4) (size 0.8) (drill 0.4) (layers F.Cu B.Cu) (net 9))
 (segment (start 133.8 57) (end 134.4 56.4) (width 0.25) (layer B.Cu) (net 9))
 (segment (start 134.4 56.4) (end 134.4 54.6) (width 0.25) (layer F.Cu) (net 9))
 (segment (start 134.4 54.6) (end 135.575 54.6) (width 0.25) (layer F.Cu) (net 9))
 (segment (start 132.8 54.6) (end 134.4 54.6) (width 0.25) (layer F.Cu) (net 9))
 (via (at 131.55213 60.796313) (size 0.8) (drill 0.4) (layers F.Cu B.Cu) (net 14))
 (segment (start 129.6375 60.875) (end 131.473443 60.875) (width 0.25) (layer F.Cu) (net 14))
 (segment (start 107 59.46) (end 107.825001 58.634999) (width 0.25) (layer B.Cu) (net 14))
 (segment (start 132.125001 60.223442) (end 131.55213 60.796313) (width 0.25) (layer B.Cu) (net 14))
 (segment (start 131.308001 58.634999) (end 132.125001 59.451999) (width 0.25) (layer B.Cu) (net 14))
 (segment (start 131.473443 60.875) (end 131.55213 60.796313) (width 0.25) (layer F.Cu) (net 14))
 (segment (start 132.125001 59.451999) (end 132.125001 60.223442) (width 0.25) (layer B.Cu) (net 14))
 (segment (start 107.825001 58.634999) (end 131.308001 58.634999) (width 0.25) (layer B.Cu) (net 14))
 (segment (start 130.949681 60.225) (end 131.387336 59.787345) (width 0.25) (layer F.Cu) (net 15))
 (segment (start 129.6375 60.225) (end 130.949681 60.225) (width 0.25) (layer F.Cu) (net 15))
 (segment (start 108.27 59.46) (end 131.059991 59.46) (width 0.25) (layer B.Cu) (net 15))
 (segment (start 131.059991 59.46) (end 131.387336 59.787345) (width 0.25) (layer B.Cu) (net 15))
 (via (at 131.387336 59.787345) (size 0.8) (drill 0.4) (layers F.Cu B.Cu) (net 15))
 (segment (start 131.494402 58.18499) (end 133 59.690588) (width 0.25) (layer B.Cu) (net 4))
 (segment (start 107.054008 58.18499) (end 131.494402 58.18499) (width 0.25) (layer B.Cu) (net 4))
 (segment (start 133.525 60.875) (end 133 61.4) (width 0.25) (layer F.Cu) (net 4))
 (segment (start 133 59.690588) (end 133 61.4) (width 0.25) (layer B.Cu) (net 4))
 (segment (start 107 60.73) (end 106.174999 59.904999) (width 0.25) (layer B.Cu) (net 4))
 (segment (start 135.3625 60.875) (end 133.525 60.875) (width 0.25) (layer F.Cu) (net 4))
 (segment (start 106.174999 59.063999) (end 107.054008 58.18499) (width 0.25) (layer B.Cu) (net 4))
 (segment (start 106.174999 59.904999) (end 106.174999 59.063999) (width 0.25) (layer B.Cu) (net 4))
 (via (at 133 61.4) (size 0.8) (drill 0.4) (layers F.Cu B.Cu) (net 4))
 (segment (start 129.6375 61.525) (end 131.119204 61.525) (width 0.25) (layer F.Cu) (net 13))
 (segment (start 131.119204 61.525) (end 131.595779 62.001575) (width 0.25) (layer F.Cu) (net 13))
 (segment (start 108.27 60.73) (end 130.324204 60.73) (width 0.25) (layer B.Cu) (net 13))
 (segment (start 130.324204 60.73) (end 131.595779 62.001575) (width 0.25) (layer B.Cu) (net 13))
 (via (at 131.595779 62.001575) (size 0.8) (drill 0.4) (layers F.Cu B.Cu) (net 13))
 (segment (start 157.575 54.05) (end 157.5 53.975) (width 0.5) (layer F.Cu) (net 5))
 (segment (start 159.5 54.05) (end 157.575 54.05) (width 0.5) (layer F.Cu) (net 5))
 (segment (start 136.525 61.525) (end 135.3625 61.525) (width 0.25) (layer F.Cu) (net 5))
 (segment (start 141.6 63.4) (end 138.4 63.4) (width 0.25) (layer F.Cu) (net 5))
 (segment (start 151.025 53.975) (end 141.6 63.4) (width 0.25) (layer F.Cu) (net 5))
 (segment (start 138.4 63.4) (end 136.525 61.525) (width 0.25) (layer F.Cu) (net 5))
 (segment (start 157.5 53.975) (end 151.025 53.975) (width 0.25) (layer F.Cu) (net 5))
 (segment (start 157.575 57.8) (end 157.5 57.725) (width 0.5) (layer F.Cu) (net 6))
 (segment (start 159.5 57.8) (end 157.575 57.8) (width 0.5) (layer F.Cu) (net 6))
 (segment (start 136.1 62.175) (end 135.3625 62.175) (width 0.25) (layer F.Cu) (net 6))
 (segment (start 138.274989 64.349989) (end 136.1 62.175) (width 0.25) (layer F.Cu) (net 6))
 (segment (start 153.574998 60.225002) (end 153.574998 62.225002) (width 0.25) (layer F.Cu) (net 6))
 (segment (start 151.450011 64.349989) (end 138.274989 64.349989) (width 0.25) (layer F.Cu) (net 6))
 (segment (start 157.5 57.725) (end 156.075 57.725) (width 0.25) (layer F.Cu) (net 6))
 (segment (start 153.574998 62.225002) (end 151.450011 64.349989) (width 0.25) (layer F.Cu) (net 6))
 (segment (start 156.075 57.725) (end 153.574998 60.225002) (width 0.25) (layer F.Cu) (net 6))
 (segment (start 135.3625 64.125) (end 134.625 64.125) (width 0.25) (layer F.Cu) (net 8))
 (segment (start 157.575 61.55) (end 157.5 61.475) (width 0.5) (layer F.Cu) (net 7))
 (segment (start 159.5 61.55) (end 157.575 61.55) (width 0.5) (layer F.Cu) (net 7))
 (segment (start 135.3625 63.475) (end 134.625 63.475) (width 0.25) (layer F.Cu) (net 7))
 (segment (start 136.475 63.475) (end 135.3625 63.475) (width 0.25) (layer F.Cu) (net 7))
 (segment (start 138 65) (end 136.475 63.475) (width 0.25) (layer F.Cu) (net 7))
 (segment (start 154.4 62.4) (end 151.8 65) (width 0.25) (layer F.Cu) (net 7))
 (segment (start 155.4 62.4) (end 154.4 62.4) (width 0.25) (layer F.Cu) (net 7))
 (segment (start 156.325 61.475) (end 155.4 62.4) (width 0.25) (layer F.Cu) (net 7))
 (segment (start 151.8 65) (end 138 65) (width 0.25) (layer F.Cu) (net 7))
 (segment (start 157.5 61.475) (end 156.325 61.475) (width 0.25) (layer F.Cu) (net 7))
 (segment (start 157.575 65.3) (end 157.5 65.225) (width 0.5) (layer F.Cu) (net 8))
 (segment (start 159.5 65.3) (end 157.575 65.3) (width 0.5) (layer F.Cu) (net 8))
 (segment (start 136.1 64.125) (end 135.3625 64.125) (width 0.25) (layer F.Cu) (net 8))
 (segment (start 137.575 65.6) (end 136.1 64.125) (width 0.25) (layer F.Cu) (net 8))
 (segment (start 157.125 65.6) (end 137.575 65.6) (width 0.25) (layer F.Cu) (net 8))
 (segment (start 157.5 65.225) (end 157.125 65.6) (width 0.25) (layer F.Cu) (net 8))
 (segment (start 106.75 56.25) (end 113 56.25) (width 1.5) (layer F.Cu) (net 17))
 (segment (start 102.5 60.5) (end 106.75 56.25) (width 1.5) (layer F.Cu) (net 17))
 (segment (start 167.75 66.25) (end 168.5 65.5) (width 1) (layer F.Cu) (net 18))
 (segment (start 161.5 66.25) (end 167.75 66.25) (width 1) (layer F.Cu) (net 18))
 (segment (start 168 62.5) (end 168.5 63) (width 1) (layer F.Cu) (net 19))
 (segment (start 161.5 62.5) (end 168 62.5) (width 1) (layer F.Cu) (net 19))
 (segment (start 163.25 60.5) (end 168.5 60.5) (width 1) (layer F.Cu) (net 20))
 (segment (start 161.5 58.75) (end 163.25 60.5) (width 1) (layer F.Cu) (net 20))
 (segment (start 164.5 58) (end 168.5 58) (width 1) (layer F.Cu) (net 21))
 (segment (start 161.5 55) (end 164.5 58) (width 1) (layer F.Cu) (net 21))
 (segment (start 112.05 58.25) (end 113.95 58.25) (width 1.5) (layer F.Cu) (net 24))
 (segment (start 112.25 58.45) (end 112.05 58.25) (width 1.5) (layer F.Cu) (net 24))
 (segment (start 112.25 60.725) (end 112.25 58.45) (width 1.5) (layer F.Cu) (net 24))
 (segment (start 113.9 60.725) (end 115.975 62.8) (width 1.5) (layer F.Cu) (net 24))
 (segment (start 112.25 60.725) (end 113.9 60.725) (width 1.5) (layer F.Cu) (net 24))
 (segment (start 115.975 64.925) (end 116 64.95) (width 1.5) (layer F.Cu) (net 24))
 (segment (start 115.975 62.8) (end 115.975 64.925) (width 1.5) (layer F.Cu) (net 24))
 (via (at 122.2 65) (size 0.8) (drill 0.4) (layers F.Cu B.Cu) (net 16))
 (segment (start 120 62.8) (end 122.2 65) (width 0.25) (layer F.Cu) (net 16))
 (segment (start 118.025 62.8) (end 120 62.8) (width 0.25) (layer F.Cu) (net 16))
 (segment (start 140.7 66.6) (end 144.6 62.7) (width 0.25) (layer B.Cu) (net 16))
 (segment (start 123.8 66.6) (end 140.7 66.6) (width 0.25) (layer B.Cu) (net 16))
 (segment (start 122.2 65) (end 123.8 66.6) (width 0.25) (layer B.Cu) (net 16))
 (segment (start 151.1 62.7) (end 144.6 62.7) (width 0.5) (layer F.Cu) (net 16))
 (segment (start 118.2 62.625) (end 118.025 62.8) (width 0.5) (layer F.Cu) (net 16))
 (segment (start 118.2 57.4) (end 118.2 62.625) (width 0.5) (layer F.Cu) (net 16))
 (segment (start 117.9 62.925) (end 118.025 62.8) (width 0.5) (layer F.Cu) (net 16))
 (segment (start 117.9 64.95) (end 117.9 62.925) (width 0.5) (layer F.Cu) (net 16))
 (segment (start 124.925 53.65) (end 122.2 56.375) (width 0.25) (layer F.Cu) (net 23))
 (segment (start 130.8 53.65) (end 124.925 53.65) (width 0.25) (layer F.Cu) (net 23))
 (segment (start 120.275 56.375) (end 120.2 56.45) (width 0.5) (layer F.Cu) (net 23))
 (segment (start 122.2 56.375) (end 120.275 56.375) (width 0.5) (layer F.Cu) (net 23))
 (via (at 122.8 62.6) (size 0.8) (drill 0.4) (layers F.Cu B.Cu) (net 10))
 (segment (start 122.2 62) (end 122.8 62.6) (width 0.25) (layer F.Cu) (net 10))
 (segment (start 122.2 58.425) (end 122.2 62) (width 0.25) (layer F.Cu) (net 10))
 (via (at 132.6 65) (size 0.8) (drill 0.4) (layers F.Cu B.Cu) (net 10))
 (segment (start 133.025 65.425) (end 135.3625 65.425) (width 0.25) (layer F.Cu) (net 10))
 (segment (start 132.6 65) (end 133.025 65.425) (width 0.25) (layer F.Cu) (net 10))
 (segment (start 130.2 62.6) (end 132.6 65) (width 0.25) (layer B.Cu) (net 10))
 (segment (start 122.8 62.6) (end 130.2 62.6) (width 0.25) (layer B.Cu) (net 10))
 (segment (start 120.275 58.425) (end 120.2 58.35) (width 0.5) (layer F.Cu) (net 10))
 (segment (start 122.2 58.425) (end 120.275 58.425) (width 0.5) (layer F.Cu) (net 10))
 (segment (start 127.225 55.55) (end 127.2 55.575) (width 0.25) (layer F.Cu) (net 22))
 (segment (start 130.8 55.55) (end 127.225 55.55) (width 0.25) (layer F.Cu) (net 22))
 (segment (start 136.225 59.575) (end 135.3625 59.575) (width 0.25) (layer F.Cu) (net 1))
 (segment (start 138.024999 57.775001) (end 136.225 59.575) (width 0.25) (layer F.Cu) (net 1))
 (segment (start 138.024999 57.089999) (end 138.024999 57.775001) (width 0.25) (layer F.Cu) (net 1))
 (segment (start 138.314998 56.8) (end 138.024999 57.089999) (width 0.25) (layer F.Cu) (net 1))
 (segment (start 140.8 56.8) (end 138.314998 56.8) (width 0.25) (layer F.Cu) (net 1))
 (segment (start 138.8 61.225) (end 138.975 61.4) (width 0.25) (layer F.Cu) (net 2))
 (segment (start 138.8 57.75) (end 138.8 61.225) (width 0.25) (layer F.Cu) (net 2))
 (segment (start 137.025 60.225) (end 135.3625 60.225) (width 0.25) (layer F.Cu) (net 2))
 (segment (start 138.2 61.4) (end 137.025 60.225) (width 0.25) (layer F.Cu) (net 2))
 (segment (start 138.975 61.4) (end 138.2 61.4) (width 0.25) (layer F.Cu) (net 2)))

